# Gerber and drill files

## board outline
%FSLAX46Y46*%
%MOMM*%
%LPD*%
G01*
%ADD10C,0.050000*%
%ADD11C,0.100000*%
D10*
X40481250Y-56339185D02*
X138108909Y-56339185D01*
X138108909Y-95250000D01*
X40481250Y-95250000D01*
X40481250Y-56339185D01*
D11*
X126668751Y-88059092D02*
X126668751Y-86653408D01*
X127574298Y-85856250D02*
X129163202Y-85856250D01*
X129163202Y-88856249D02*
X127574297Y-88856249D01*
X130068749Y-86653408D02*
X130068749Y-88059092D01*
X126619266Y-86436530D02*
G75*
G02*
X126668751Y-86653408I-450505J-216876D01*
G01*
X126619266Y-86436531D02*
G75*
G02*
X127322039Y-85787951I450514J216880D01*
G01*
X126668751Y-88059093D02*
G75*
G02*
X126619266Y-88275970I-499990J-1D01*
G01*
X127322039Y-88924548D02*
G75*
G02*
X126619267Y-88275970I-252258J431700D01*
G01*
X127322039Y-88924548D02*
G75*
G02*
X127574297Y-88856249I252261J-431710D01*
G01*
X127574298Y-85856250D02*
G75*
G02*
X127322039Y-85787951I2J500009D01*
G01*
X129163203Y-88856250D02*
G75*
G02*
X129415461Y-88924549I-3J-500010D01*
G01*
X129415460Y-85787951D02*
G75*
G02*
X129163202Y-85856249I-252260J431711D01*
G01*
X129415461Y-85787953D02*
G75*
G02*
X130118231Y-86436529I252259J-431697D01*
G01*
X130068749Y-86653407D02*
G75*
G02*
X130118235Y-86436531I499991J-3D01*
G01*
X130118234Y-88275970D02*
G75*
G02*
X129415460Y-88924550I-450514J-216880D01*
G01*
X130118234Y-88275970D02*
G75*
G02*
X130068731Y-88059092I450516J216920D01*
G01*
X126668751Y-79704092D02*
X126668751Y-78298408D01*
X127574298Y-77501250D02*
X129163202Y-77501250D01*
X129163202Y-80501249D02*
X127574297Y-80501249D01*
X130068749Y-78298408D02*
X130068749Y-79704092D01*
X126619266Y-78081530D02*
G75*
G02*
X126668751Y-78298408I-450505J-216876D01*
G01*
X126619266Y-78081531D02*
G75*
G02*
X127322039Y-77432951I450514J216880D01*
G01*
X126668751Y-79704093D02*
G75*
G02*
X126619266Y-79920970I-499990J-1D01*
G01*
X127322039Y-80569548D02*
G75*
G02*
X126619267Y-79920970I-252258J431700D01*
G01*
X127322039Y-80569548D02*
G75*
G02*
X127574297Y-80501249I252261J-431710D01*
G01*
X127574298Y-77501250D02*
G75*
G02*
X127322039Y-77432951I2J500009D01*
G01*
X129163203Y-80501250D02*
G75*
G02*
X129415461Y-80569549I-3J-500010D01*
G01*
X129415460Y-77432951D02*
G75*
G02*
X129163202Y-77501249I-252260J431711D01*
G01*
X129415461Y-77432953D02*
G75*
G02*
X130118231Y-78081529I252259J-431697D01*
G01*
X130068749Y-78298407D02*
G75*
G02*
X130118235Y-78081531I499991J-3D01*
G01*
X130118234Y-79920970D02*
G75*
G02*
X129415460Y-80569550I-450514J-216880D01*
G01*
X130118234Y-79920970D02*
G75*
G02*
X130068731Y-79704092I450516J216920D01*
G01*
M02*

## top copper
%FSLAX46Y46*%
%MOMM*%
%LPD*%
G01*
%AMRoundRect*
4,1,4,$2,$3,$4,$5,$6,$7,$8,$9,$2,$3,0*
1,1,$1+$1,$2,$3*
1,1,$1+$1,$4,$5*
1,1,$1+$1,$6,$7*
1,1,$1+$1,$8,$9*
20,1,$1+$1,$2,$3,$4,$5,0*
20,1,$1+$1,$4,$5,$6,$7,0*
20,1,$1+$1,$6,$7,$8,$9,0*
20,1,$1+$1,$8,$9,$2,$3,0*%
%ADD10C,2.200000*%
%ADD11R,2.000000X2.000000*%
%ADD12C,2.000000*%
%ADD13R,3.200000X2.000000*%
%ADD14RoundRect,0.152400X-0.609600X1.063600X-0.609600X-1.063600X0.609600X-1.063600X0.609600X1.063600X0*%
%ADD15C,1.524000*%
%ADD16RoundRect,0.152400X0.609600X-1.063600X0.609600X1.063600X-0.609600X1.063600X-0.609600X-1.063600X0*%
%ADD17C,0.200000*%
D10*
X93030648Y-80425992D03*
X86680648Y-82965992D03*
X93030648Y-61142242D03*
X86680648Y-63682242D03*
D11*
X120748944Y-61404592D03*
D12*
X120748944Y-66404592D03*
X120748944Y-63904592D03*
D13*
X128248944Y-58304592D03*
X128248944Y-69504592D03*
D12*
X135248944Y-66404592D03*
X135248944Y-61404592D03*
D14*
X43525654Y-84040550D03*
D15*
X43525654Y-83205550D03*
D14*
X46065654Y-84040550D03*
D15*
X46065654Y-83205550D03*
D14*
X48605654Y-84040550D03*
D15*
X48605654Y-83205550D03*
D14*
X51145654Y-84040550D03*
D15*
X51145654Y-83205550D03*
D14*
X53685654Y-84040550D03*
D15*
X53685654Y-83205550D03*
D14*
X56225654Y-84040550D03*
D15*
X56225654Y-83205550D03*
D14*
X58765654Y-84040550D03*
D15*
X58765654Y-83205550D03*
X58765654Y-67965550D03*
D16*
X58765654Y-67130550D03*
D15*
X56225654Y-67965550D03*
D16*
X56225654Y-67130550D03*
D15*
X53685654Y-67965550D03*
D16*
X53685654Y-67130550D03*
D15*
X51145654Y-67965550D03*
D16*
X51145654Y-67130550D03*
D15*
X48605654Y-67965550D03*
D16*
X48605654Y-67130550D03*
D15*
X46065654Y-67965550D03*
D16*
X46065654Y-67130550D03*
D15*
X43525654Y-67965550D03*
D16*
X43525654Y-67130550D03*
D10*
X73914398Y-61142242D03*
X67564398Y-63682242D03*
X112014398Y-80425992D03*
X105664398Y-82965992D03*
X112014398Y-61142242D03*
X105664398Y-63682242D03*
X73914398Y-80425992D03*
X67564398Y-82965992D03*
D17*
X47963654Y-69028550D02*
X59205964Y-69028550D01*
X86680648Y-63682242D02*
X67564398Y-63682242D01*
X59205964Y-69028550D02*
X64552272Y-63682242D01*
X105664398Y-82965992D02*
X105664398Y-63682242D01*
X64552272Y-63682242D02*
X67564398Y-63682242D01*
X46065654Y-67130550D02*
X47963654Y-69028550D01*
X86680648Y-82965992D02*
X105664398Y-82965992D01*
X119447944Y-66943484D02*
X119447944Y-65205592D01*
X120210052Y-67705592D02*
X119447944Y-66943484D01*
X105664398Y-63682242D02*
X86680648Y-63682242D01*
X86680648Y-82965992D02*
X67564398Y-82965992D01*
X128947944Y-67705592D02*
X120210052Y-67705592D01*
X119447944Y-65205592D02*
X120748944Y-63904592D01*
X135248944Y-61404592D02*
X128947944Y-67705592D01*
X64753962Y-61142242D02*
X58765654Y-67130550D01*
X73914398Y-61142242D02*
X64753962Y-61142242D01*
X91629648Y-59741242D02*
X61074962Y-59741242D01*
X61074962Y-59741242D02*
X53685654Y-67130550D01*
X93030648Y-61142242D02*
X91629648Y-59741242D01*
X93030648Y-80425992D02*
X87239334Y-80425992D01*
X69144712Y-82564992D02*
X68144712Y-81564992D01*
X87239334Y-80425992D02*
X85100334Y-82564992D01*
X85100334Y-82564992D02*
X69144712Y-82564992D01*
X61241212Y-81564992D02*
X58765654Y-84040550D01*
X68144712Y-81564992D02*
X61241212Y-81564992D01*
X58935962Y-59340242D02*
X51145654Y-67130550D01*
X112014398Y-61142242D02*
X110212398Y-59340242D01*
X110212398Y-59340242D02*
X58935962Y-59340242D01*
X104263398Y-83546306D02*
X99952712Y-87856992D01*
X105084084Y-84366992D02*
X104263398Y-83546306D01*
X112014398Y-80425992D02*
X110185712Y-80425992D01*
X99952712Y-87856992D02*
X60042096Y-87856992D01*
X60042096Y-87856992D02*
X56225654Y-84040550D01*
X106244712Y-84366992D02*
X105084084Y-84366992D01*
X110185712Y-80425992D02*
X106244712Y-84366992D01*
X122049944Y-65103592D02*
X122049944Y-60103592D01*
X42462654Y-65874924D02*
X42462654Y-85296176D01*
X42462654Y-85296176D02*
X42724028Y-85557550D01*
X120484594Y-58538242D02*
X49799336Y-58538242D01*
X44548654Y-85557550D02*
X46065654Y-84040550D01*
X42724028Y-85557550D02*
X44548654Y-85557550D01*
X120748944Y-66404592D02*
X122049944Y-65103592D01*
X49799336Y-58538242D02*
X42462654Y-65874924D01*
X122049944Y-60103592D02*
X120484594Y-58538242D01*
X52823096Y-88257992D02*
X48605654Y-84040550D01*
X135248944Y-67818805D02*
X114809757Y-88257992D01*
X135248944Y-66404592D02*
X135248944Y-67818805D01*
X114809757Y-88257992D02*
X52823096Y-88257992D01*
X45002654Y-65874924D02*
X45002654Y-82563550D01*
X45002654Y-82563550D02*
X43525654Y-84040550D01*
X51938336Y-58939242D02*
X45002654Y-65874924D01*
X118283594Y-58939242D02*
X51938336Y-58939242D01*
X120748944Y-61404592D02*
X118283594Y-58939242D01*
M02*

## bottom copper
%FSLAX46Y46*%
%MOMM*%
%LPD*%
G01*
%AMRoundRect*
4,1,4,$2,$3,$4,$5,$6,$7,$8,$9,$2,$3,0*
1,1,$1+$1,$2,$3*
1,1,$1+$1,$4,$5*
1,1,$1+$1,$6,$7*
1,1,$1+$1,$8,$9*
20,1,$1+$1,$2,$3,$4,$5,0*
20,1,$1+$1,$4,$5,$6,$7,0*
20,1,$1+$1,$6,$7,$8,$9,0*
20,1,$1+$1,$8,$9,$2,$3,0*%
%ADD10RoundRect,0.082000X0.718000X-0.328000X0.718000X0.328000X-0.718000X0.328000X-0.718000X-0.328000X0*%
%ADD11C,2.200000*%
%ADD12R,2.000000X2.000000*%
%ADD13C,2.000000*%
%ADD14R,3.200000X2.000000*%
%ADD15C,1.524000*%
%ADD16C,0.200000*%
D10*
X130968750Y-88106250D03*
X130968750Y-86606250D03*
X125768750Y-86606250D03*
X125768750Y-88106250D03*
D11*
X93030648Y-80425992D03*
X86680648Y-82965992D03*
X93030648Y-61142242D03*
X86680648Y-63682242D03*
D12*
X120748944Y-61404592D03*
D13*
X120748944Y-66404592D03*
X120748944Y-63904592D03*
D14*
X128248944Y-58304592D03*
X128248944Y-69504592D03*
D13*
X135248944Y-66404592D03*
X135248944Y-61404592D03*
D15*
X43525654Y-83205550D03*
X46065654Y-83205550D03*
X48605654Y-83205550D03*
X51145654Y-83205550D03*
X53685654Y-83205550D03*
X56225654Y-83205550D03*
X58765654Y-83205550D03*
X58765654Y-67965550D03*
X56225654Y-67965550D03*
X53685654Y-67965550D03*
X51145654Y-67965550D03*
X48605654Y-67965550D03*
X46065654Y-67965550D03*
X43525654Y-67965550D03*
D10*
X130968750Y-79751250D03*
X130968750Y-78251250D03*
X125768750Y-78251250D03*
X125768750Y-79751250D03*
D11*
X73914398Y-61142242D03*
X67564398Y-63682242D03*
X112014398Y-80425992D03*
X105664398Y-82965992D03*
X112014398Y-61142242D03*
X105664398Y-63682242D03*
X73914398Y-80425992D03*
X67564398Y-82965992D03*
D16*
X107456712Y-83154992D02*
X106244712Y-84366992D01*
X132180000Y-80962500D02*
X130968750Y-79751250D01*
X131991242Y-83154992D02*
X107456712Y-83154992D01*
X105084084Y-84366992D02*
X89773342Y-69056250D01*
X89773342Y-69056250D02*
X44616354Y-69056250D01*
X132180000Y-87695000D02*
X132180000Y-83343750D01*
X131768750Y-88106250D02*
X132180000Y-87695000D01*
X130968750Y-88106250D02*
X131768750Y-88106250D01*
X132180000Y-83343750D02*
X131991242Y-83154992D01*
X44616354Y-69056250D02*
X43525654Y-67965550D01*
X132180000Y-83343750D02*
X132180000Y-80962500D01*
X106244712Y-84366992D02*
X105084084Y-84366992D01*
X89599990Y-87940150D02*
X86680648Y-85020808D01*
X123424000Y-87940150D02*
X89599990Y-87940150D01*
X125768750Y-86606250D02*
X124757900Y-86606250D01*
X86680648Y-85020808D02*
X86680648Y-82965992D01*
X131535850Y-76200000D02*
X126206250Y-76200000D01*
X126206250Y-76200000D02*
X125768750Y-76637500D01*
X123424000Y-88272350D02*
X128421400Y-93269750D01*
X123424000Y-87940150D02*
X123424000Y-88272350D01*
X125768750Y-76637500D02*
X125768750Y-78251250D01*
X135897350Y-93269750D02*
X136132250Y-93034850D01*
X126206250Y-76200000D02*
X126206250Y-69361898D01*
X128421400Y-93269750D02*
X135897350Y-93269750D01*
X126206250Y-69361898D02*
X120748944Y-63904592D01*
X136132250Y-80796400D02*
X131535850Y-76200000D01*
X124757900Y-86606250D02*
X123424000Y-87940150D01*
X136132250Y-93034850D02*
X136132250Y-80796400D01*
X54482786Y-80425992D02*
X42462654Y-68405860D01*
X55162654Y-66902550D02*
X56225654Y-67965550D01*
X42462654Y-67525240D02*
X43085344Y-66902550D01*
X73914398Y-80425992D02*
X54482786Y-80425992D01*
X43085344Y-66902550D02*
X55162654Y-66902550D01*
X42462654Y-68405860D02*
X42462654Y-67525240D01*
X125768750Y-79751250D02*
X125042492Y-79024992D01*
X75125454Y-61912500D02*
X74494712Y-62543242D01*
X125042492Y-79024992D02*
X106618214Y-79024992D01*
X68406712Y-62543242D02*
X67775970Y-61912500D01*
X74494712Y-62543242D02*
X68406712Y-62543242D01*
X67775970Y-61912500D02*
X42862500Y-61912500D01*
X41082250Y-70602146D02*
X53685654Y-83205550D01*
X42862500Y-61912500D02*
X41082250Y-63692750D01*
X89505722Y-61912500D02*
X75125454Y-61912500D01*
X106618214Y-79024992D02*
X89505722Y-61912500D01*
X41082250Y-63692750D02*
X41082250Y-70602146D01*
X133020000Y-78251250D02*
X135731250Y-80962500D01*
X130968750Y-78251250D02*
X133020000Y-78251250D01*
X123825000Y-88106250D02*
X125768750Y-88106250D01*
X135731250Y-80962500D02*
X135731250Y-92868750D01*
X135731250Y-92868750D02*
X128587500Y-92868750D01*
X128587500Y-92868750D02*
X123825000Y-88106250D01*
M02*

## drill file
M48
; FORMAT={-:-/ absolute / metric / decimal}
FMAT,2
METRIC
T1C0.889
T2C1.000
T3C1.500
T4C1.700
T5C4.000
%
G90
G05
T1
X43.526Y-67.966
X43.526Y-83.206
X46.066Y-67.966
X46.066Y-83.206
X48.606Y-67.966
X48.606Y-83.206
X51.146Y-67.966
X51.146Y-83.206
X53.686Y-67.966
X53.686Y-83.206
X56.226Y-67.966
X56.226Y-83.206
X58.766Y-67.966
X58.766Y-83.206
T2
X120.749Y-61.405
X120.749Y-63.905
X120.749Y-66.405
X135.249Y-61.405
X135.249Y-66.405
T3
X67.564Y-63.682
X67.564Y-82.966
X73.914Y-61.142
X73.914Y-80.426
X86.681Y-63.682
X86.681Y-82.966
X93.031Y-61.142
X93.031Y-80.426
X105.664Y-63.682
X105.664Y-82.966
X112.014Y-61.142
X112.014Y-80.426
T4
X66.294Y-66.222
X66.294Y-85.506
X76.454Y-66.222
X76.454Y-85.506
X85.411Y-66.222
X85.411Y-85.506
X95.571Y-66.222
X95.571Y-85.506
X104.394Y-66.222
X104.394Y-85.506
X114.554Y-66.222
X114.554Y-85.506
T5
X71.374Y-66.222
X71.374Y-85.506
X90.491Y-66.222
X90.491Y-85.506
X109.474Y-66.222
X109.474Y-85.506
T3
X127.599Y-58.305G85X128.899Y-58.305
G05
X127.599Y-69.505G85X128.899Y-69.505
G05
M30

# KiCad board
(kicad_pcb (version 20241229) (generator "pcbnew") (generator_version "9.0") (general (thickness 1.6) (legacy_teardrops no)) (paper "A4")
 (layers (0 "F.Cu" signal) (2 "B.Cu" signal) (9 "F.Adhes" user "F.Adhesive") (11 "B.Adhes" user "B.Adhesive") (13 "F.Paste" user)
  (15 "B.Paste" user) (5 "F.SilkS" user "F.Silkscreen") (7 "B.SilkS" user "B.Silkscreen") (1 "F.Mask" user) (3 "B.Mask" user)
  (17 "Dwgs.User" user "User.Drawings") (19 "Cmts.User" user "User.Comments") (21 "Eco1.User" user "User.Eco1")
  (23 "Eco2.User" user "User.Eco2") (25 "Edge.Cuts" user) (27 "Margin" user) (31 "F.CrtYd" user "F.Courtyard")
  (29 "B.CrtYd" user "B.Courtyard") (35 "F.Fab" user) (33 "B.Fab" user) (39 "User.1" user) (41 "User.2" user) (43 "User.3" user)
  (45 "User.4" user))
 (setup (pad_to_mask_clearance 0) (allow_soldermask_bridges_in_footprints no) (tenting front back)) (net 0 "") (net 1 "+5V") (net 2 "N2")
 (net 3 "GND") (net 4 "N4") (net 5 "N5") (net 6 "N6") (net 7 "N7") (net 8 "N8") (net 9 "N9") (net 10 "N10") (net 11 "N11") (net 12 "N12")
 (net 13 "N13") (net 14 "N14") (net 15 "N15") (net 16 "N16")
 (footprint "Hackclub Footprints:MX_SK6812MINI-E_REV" (layer "F.Cu") (at 128.36875 82.27625)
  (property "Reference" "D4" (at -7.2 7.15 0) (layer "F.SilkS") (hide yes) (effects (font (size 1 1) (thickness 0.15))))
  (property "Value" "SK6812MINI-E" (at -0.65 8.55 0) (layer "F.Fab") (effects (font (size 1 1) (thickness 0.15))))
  (fp_line (start -1.699999 5.782842) (end -1.699999 4.377158) (stroke (width 0.1) (type solid)) (layer "Edge.Cuts"))
  (fp_line (start -0.794452 3.58) (end 0.794452 3.58) (stroke (width 0.1) (type solid)) (layer "Edge.Cuts"))
  (fp_line (start 0.794452 6.579999) (end -0.794453 6.579999) (stroke (width 0.1) (type solid)) (layer "Edge.Cuts"))
  (fp_line (start 1.699999 4.377158) (end 1.699999 5.782842) (stroke (width 0.1) (type solid)) (layer "Edge.Cuts"))
  (fp_arc (start -1.749484 4.16028) (mid -1.712527 4.265932) (end -1.699999 4.377158) (stroke (width 0.1) (type solid)) (layer "Edge.Cuts"))
  (fp_arc (start -1.749484 4.160281) (mid -1.638072 3.575965) (end -1.046711 3.511701) (stroke (width 0.1) (type solid)) (layer "Edge.Cuts"))
  (fp_arc (start -1.699999 5.782843) (mid -1.712527 5.894068) (end -1.749484 5.99972) (stroke (width 0.1) (type solid)) (layer "Edge.Cuts"))
  (fp_arc (start -1.046711 6.648298) (mid -1.638071 6.584034) (end -1.749484 5.99972) (stroke (width 0.1) (type solid)) (layer "Edge.Cuts"))
  (fp_arc (start -1.046711 6.648298) (mid -0.925123 6.597376) (end -0.794453 6.579999) (stroke (width 0.1) (type solid)) (layer "Edge.Cuts"))
  (fp_arc (start -0.794452 3.58) (mid -0.925123 3.562623) (end -1.046711 3.511701) (stroke (width 0.1) (type solid)) (layer "Edge.Cuts"))
  (fp_arc (start 0.794453 6.58) (mid 0.925123 6.597377) (end 1.046711 6.648299) (stroke (width 0.1) (type solid)) (layer "Edge.Cuts"))
  (fp_arc (start 1.04671 3.511701) (mid 0.925122 3.562623) (end 0.794452 3.58) (stroke (width 0.1) (type solid)) (layer "Edge.Cuts"))
  (fp_arc (start 1.046711 3.511703) (mid 1.63807 3.575966) (end 1.749484 4.16028) (stroke (width 0.1) (type solid)) (layer "Edge.Cuts"))
  (fp_arc (start 1.699999 4.377157) (mid 1.712527 4.265932) (end 1.749484 4.16028) (stroke (width 0.1) (type solid)) (layer "Edge.Cuts"))
  (fp_arc (start 1.749484 5.99972) (mid 1.638071 6.584035) (end 1.046711 6.648299) (stroke (width 0.1) (type solid)) (layer "Edge.Cuts"))
  (fp_arc (start 1.749484 5.99972) (mid 1.712527 5.894068) (end 1.699999 5.782842) (stroke (width 0.1) (type solid)) (layer "Edge.Cuts"))
  (pad "1" smd roundrect (at 2.6 5.83 90) (size 0.82 1.6) (layers "B.Cu" "B.Mask" "B.Paste") (roundrect_rratio 0.1) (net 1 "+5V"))
  (pad "2" smd roundrect (at 2.6 4.33 90) (size 0.82 1.6) (layers "B.Cu" "B.Mask" "B.Paste") (roundrect_rratio 0.1) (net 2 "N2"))
  (pad "3" smd roundrect (at -2.6 4.33 90) (size 0.82 1.6) (layers "B.Cu" "B.Mask" "B.Paste") (roundrect_rratio 0.1) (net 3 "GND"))
  (pad "4" smd roundrect (at -2.6 5.83 90) (size 0.82 1.6) (layers "B.Cu" "B.Mask" "B.Paste") (roundrect_rratio 0.1) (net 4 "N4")))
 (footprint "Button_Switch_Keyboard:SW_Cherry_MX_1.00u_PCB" (layer "F.Cu") (at 93.030648 80.425992)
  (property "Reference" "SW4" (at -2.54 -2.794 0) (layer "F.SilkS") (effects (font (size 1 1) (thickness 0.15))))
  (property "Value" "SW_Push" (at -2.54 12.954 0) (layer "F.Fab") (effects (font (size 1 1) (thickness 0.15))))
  (pad "" np_thru_hole circle (at -7.62 5.08) (size 1.7 1.7) (drill 1.7) (layers "*.Cu" "*.Mask"))
  (pad "" np_thru_hole circle (at -2.54 5.08) (size 4 4) (drill 4) (layers "*.Cu" "*.Mask"))
  (pad "" np_thru_hole circle (at 2.54 5.08) (size 1.7 1.7) (drill 1.7) (layers "*.Cu" "*.Mask"))
  (pad "1" thru_hole circle (at 0 0) (size 2.2 2.2) (drill 1.5) (layers "*.Cu" "*.Mask") (remove_unused_layers no) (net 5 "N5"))
  (pad "2" thru_hole circle (at -6.35 2.54) (size 2.2 2.2) (drill 1.5) (layers "*.Cu" "*.Mask") (remove_unused_layers no) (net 3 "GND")))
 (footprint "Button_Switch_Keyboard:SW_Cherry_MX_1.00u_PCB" (layer "F.Cu") (at 93.030648 61.142242)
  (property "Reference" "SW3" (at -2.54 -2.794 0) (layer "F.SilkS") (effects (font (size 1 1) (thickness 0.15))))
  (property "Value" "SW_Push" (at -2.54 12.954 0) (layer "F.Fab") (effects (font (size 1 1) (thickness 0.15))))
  (pad "" np_thru_hole circle (at -7.62 5.08) (size 1.7 1.7) (drill 1.7) (layers "*.Cu" "*.Mask"))
  (pad "" np_thru_hole circle (at -2.54 5.08) (size 4 4) (drill 4) (layers "*.Cu" "*.Mask"))
  (pad "" np_thru_hole circle (at 2.54 5.08) (size 1.7 1.7) (drill 1.7) (layers "*.Cu" "*.Mask"))
  (pad "1" thru_hole circle (at 0 0) (size 2.2 2.2) (drill 1.5) (layers "*.Cu" "*.Mask") (remove_unused_layers no) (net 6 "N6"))
  (pad "2" thru_hole circle (at -6.35 2.54) (size 2.2 2.2) (drill 1.5) (layers "*.Cu" "*.Mask") (remove_unused_layers no) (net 3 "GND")))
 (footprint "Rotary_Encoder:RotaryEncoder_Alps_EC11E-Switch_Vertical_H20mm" (layer "F.Cu") (at 120.748944 61.404592)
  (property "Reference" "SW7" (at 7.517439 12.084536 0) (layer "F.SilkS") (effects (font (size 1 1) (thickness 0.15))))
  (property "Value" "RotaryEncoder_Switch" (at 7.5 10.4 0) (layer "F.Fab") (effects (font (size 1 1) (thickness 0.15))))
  (pad "A" thru_hole rect (at 0 0) (size 2 2) (drill 1) (layers "*.Cu" "*.Mask") (remove_unused_layers no) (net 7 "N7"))
  (pad "B" thru_hole circle (at 0 5) (size 2 2) (drill 1) (layers "*.Cu" "*.Mask") (remove_unused_layers no) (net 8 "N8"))
  (pad "C" thru_hole circle (at 0 2.5) (size 2 2) (drill 1) (layers "*.Cu" "*.Mask") (remove_unused_layers no) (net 3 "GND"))
  (pad "MP" thru_hole rect (at 7.5 -3.1) (size 3.2 2) (drill oval 2.8 1.5) (layers "*.Cu" "*.Mask") (remove_unused_layers no))
  (pad "MP" thru_hole rect (at 7.5 8.1) (size 3.2 2) (drill oval 2.8 1.5) (layers "*.Cu" "*.Mask") (remove_unused_layers no))
  (pad "S1" thru_hole circle (at 14.5 5) (size 2 2) (drill 1) (layers "*.Cu" "*.Mask") (remove_unused_layers no) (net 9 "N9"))
  (pad "S2" thru_hole circle (at 14.5 0) (size 2 2) (drill 1) (layers "*.Cu" "*.Mask") (remove_unused_layers no) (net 3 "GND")))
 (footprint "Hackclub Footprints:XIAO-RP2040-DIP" (layer "F.Cu") (at 51.145654 75.58555 90)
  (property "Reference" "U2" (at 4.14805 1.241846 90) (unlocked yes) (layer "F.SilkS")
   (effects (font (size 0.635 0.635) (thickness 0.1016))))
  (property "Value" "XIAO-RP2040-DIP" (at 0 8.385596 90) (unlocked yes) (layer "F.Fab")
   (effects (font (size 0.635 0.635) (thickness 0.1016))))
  (pad "1" smd roundrect (at -8.455 -7.62 270) (size 2.432 1.524) (layers "F.Cu" "F.Mask") (roundrect_rratio 0.1) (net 7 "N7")
   (thermal_bridge_angle 45))
  (pad "1" thru_hole circle (at -7.62 -7.62 270) (size 1.524 1.524) (drill 0.889) (layers "*.Cu" "*.Mask") (remove_unused_layers no)
   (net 7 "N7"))
  (pad "2" smd roundrect (at -8.455 -5.08 270) (size 2.432 1.524) (layers "F.Cu" "F.Mask") (roundrect_rratio 0.1) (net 8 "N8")
   (thermal_bridge_angle 45))
  (pad "2" thru_hole circle (at -7.62 -5.08 270) (size 1.524 1.524) (drill 0.889) (layers "*.Cu" "*.Mask") (remove_unused_layers no)
   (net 8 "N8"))
  (pad "3" smd roundrect (at -8.455 -2.54 270) (size 2.432 1.524) (layers "F.Cu" "F.Mask") (roundrect_rratio 0.1) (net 9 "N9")
   (thermal_bridge_angle 45))
  (pad "3" thru_hole circle (at -7.62 -2.54 270) (size 1.524 1.524) (drill 0.889) (layers "*.Cu" "*.Mask") (remove_unused_layers no)
   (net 9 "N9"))
  (pad "4" smd roundrect (at -8.455 0 270) (size 2.432 1.524) (layers "F.Cu" "F.Mask") (roundrect_rratio 0.1) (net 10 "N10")
   (thermal_bridge_angle 45))
  (pad "4" thru_hole circle (at -7.62 0 270) (size 1.524 1.524) (drill 0.889) (layers "*.Cu" "*.Mask") (remove_unused_layers no)
   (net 10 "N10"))
  (pad "5" smd roundrect (at -8.455 2.54 270) (size 2.432 1.524) (layers "F.Cu" "F.Mask") (roundrect_rratio 0.1) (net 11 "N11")
   (thermal_bridge_angle 45))
  (pad "5" thru_hole circle (at -7.62 2.54 270) (size 1.524 1.524) (drill 0.889) (layers "*.Cu" "*.Mask") (remove_unused_layers no)
   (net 11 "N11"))
  (pad "6" smd roundrect (at -8.455 5.08 270) (size 2.432 1.524) (layers "F.Cu" "F.Mask") (roundrect_rratio 0.1) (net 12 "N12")
   (thermal_bridge_angle 45))
  (pad "6" thru_hole circle (at -7.62 5.08 270) (size 1.524 1.524) (drill 0.889) (layers "*.Cu" "*.Mask") (remove_unused_layers no)
   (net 12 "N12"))
  (pad "7" smd roundrect (at -8.455 7.62 270) (size 2.432 1.524) (layers "F.Cu" "F.Mask") (roundrect_rratio 0.1) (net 5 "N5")
   (thermal_bridge_angle 45))
  (pad "7" thru_hole circle (at -7.62 7.62 270) (size 1.524 1.524) (drill 0.889) (layers "*.Cu" "*.Mask") (remove_unused_layers no)
   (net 5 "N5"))
  (pad "8" thru_hole circle (at 7.62 7.62 90) (size 1.524 1.524) (drill 0.889) (layers "*.Cu" "*.Mask") (remove_unused_layers no)
   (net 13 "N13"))
  (pad "8" smd roundrect (at 8.455 7.62 90) (size 2.432 1.524) (layers "F.Cu" "F.Mask") (roundrect_rratio 0.1) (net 13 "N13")
   (thermal_bridge_angle 45))
  (pad "9" thru_hole circle (at 7.62 5.08 90) (size 1.524 1.524) (drill 0.889) (layers "*.Cu" "*.Mask") (remove_unused_layers no)
   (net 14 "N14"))
  (pad "9" smd roundrect (at 8.455 5.08 90) (size 2.432 1.524) (layers "F.Cu" "F.Mask") (roundrect_rratio 0.1) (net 14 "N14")
   (thermal_bridge_angle 45))
  (pad "10" thru_hole circle (at 7.62 2.54 90) (size 1.524 1.524) (drill 0.889) (layers "*.Cu" "*.Mask") (remove_unused_layers no)
   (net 6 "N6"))
  (pad "10" smd roundrect (at 8.455 2.54 90) (size 2.432 1.524) (layers "F.Cu" "F.Mask") (roundrect_rratio 0.1) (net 6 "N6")
   (thermal_bridge_angle 45))
  (pad "11" thru_hole circle (at 7.62 0 90) (size 1.524 1.524) (drill 0.889) (layers "*.Cu" "*.Mask") (remove_unused_layers no)
   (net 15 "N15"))
  (pad "11" smd roundrect (at 8.455 0 90) (size 2.432 1.524) (layers "F.Cu" "F.Mask") (roundrect_rratio 0.1) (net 15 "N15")
   (thermal_bridge_angle 45))
  (pad "12" thru_hole circle (at 7.62 -2.54 90) (size 1.524 1.524) (drill 0.889) (layers "*.Cu" "*.Mask") (remove_unused_layers no)
   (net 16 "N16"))
  (pad "12" smd roundrect (at 8.455 -2.54 90) (size 2.432 1.524) (layers "F.Cu" "F.Mask") (roundrect_rratio 0.1) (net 16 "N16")
   (thermal_bridge_angle 45))
  (pad "13" thru_hole circle (at 7.62 -5.08 90) (size 1.524 1.524) (drill 0.889) (layers "*.Cu" "*.Mask") (remove_unused_layers no)
   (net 3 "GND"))
  (pad "13" smd roundrect (at 8.455 -5.08 90) (size 2.432 1.524) (layers "F.Cu" "F.Mask") (roundrect_rratio 0.1) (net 3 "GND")
   (thermal_bridge_angle 45))
  (pad "14" thru_hole circle (at 7.62 -7.62 90) (size 1.524 1.524) (drill 0.889) (layers "*.Cu" "*.Mask") (remove_unused_layers no)
   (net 1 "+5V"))
  (pad "14" smd roundrect (at 8.455 -7.62 90) (size 2.432 1.524) (layers "F.Cu" "F.Mask") (roundrect_rratio 0.1) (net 1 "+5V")
   (thermal_bridge_angle 45)))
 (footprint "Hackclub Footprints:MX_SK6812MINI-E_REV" (layer "F.Cu") (at 128.36875 73.92125)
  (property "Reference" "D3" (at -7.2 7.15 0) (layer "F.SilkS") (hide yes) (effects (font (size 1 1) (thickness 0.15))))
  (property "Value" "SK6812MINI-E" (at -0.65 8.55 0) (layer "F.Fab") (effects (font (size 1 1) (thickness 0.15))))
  (fp_line (start -1.699999 5.782842) (end -1.699999 4.377158) (stroke (width 0.1) (type solid)) (layer "Edge.Cuts"))
  (fp_line (start -0.794452 3.58) (end 0.794452 3.58) (stroke (width 0.1) (type solid)) (layer "Edge.Cuts"))
  (fp_line (start 0.794452 6.579999) (end -0.794453 6.579999) (stroke (width 0.1) (type solid)) (layer "Edge.Cuts"))
  (fp_line (start 1.699999 4.377158) (end 1.699999 5.782842) (stroke (width 0.1) (type solid)) (layer "Edge.Cuts"))
  (fp_arc (start -1.749484 4.16028) (mid -1.712527 4.265932) (end -1.699999 4.377158) (stroke (width 0.1) (type solid)) (layer "Edge.Cuts"))
  (fp_arc (start -1.749484 4.160281) (mid -1.638072 3.575965) (end -1.046711 3.511701) (stroke (width 0.1) (type solid)) (layer "Edge.Cuts"))
  (fp_arc (start -1.699999 5.782843) (mid -1.712527 5.894068) (end -1.749484 5.99972) (stroke (width 0.1) (type solid)) (layer "Edge.Cuts"))
  (fp_arc (start -1.046711 6.648298) (mid -1.638071 6.584034) (end -1.749484 5.99972) (stroke (width 0.1) (type solid)) (layer "Edge.Cuts"))
  (fp_arc (start -1.046711 6.648298) (mid -0.925123 6.597376) (end -0.794453 6.579999) (stroke (width 0.1) (type solid)) (layer "Edge.Cuts"))
  (fp_arc (start -0.794452 3.58) (mid -0.925123 3.562623) (end -1.046711 3.511701) (stroke (width 0.1) (type solid)) (layer "Edge.Cuts"))
  (fp_arc (start 0.794453 6.58) (mid 0.925123 6.597377) (end 1.046711 6.648299) (stroke (width 0.1) (type solid)) (layer "Edge.Cuts"))
  (fp_arc (start 1.04671 3.511701) (mid 0.925122 3.562623) (end 0.794452 3.58) (stroke (width 0.1) (type solid)) (layer "Edge.Cuts"))
  (fp_arc (start 1.046711 3.511703) (mid 1.63807 3.575966) (end 1.749484 4.16028) (stroke (width 0.1) (type solid)) (layer "Edge.Cuts"))
  (fp_arc (start 1.699999 4.377157) (mid 1.712527 4.265932) (end 1.749484 4.16028) (stroke (width 0.1) (type solid)) (layer "Edge.Cuts"))
  (fp_arc (start 1.749484 5.99972) (mid 1.638071 6.584035) (end 1.046711 6.648299) (stroke (width 0.1) (type solid)) (layer "Edge.Cuts"))
  (fp_arc (start 1.749484 5.99972) (mid 1.712527 5.894068) (end 1.699999 5.782842) (stroke (width 0.1) (type solid)) (layer "Edge.Cuts"))
  (pad "1" smd roundrect (at 2.6 5.83 90) (size 0.82 1.6) (layers "B.Cu" "B.Mask" "B.Paste") (roundrect_rratio 0.1) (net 1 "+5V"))
  (pad "2" smd roundrect (at 2.6 4.33 90) (size 0.82 1.6) (layers "B.Cu" "B.Mask" "B.Paste") (roundrect_rratio 0.1) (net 4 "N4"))
  (pad "3" smd roundrect (at -2.6 4.33 90) (size 0.82 1.6) (layers "B.Cu" "B.Mask" "B.Paste") (roundrect_rratio 0.1) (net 3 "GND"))
  (pad "4" smd roundrect (at -2.6 5.83 90) (size 0.82 1.6) (layers "B.Cu" "B.Mask" "B.Paste") (roundrect_rratio 0.1) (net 11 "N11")))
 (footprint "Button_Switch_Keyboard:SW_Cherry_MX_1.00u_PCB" (layer "F.Cu") (at 73.914398 61.142242)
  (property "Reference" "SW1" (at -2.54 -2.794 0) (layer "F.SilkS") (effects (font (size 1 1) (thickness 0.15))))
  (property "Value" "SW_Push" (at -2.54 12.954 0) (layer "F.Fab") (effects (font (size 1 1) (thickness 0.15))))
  (pad "" np_thru_hole circle (at -7.62 5.08) (size 1.7 1.7) (drill 1.7) (layers "*.Cu" "*.Mask"))
  (pad "" np_thru_hole circle (at -2.54 5.08) (size 4 4) (drill 4) (layers "*.Cu" "*.Mask"))
  (pad "" np_thru_hole circle (at 2.54 5.08) (size 1.7 1.7) (drill 1.7) (layers "*.Cu" "*.Mask"))
  (pad "1" thru_hole circle (at 0 0) (size 2.2 2.2) (drill 1.5) (layers "*.Cu" "*.Mask") (remove_unused_layers no) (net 13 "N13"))
  (pad "2" thru_hole circle (at -6.35 2.54) (size 2.2 2.2) (drill 1.5) (layers "*.Cu" "*.Mask") (remove_unused_layers no) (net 3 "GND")))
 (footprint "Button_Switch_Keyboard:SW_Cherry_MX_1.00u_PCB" (layer "F.Cu") (at 112.014398 80.425992)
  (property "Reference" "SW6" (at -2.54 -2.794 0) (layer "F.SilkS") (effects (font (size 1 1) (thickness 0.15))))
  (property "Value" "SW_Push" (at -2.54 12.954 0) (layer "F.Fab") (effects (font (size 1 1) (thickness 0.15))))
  (pad "" np_thru_hole circle (at -7.62 5.08) (size 1.7 1.7) (drill 1.7) (layers "*.Cu" "*.Mask"))
  (pad "" np_thru_hole circle (at -2.54 5.08) (size 4 4) (drill 4) (layers "*.Cu" "*.Mask"))
  (pad "" np_thru_hole circle (at 2.54 5.08) (size 1.7 1.7) (drill 1.7) (layers "*.Cu" "*.Mask"))
  (pad "1" thru_hole circle (at 0 0) (size 2.2 2.2) (drill 1.5) (layers "*.Cu" "*.Mask") (remove_unused_layers no) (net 12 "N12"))
  (pad "2" thru_hole circle (at -6.35 2.54) (size 2.2 2.2) (drill 1.5) (layers "*.Cu" "*.Mask") (remove_unused_layers no) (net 3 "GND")))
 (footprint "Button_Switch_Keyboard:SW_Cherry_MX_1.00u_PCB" (layer "F.Cu") (at 112.014398 61.142242)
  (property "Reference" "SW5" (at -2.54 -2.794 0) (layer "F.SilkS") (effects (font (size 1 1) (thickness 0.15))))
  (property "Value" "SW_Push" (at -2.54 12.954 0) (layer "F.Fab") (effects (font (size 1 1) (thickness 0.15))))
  (pad "" np_thru_hole circle (at -7.62 5.08) (size 1.7 1.7) (drill 1.7) (layers "*.Cu" "*.Mask"))
  (pad "" np_thru_hole circle (at -2.54 5.08) (size 4 4) (drill 4) (layers "*.Cu" "*.Mask"))
  (pad "" np_thru_hole circle (at 2.54 5.08) (size 1.7 1.7) (drill 1.7) (layers "*.Cu" "*.Mask"))
  (pad "1" thru_hole circle (at 0 0) (size 2.2 2.2) (drill 1.5) (layers "*.Cu" "*.Mask") (remove_unused_layers no) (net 15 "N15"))
  (pad "2" thru_hole circle (at -6.35 2.54) (size 2.2 2.2) (drill 1.5) (layers "*.Cu" "*.Mask") (remove_unused_layers no) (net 3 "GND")))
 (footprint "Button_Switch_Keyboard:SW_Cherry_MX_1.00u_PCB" (layer "F.Cu") (at 73.914398 80.425992)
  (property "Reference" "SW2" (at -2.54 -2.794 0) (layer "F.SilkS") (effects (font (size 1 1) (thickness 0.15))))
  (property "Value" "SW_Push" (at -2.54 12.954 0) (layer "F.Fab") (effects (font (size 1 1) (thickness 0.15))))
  (pad "" np_thru_hole circle (at -7.62 5.08) (size 1.7 1.7) (drill 1.7) (layers "*.Cu" "*.Mask"))
  (pad "" np_thru_hole circle (at -2.54 5.08) (size 4 4) (drill 4) (layers "*.Cu" "*.Mask"))
  (pad "" np_thru_hole circle (at 2.54 5.08) (size 1.7 1.7) (drill 1.7) (layers "*.Cu" "*.Mask"))
  (pad "1" thru_hole circle (at 0 0) (size 2.2 2.2) (drill 1.5) (layers "*.Cu" "*.Mask") (remove_unused_layers no) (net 14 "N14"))
  (pad "2" thru_hole circle (at -6.35 2.54) (size 2.2 2.2) (drill 1.5) (layers "*.Cu" "*.Mask") (remove_unused_layers no) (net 3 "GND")))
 (gr_rect (start 40.48125 56.339185) (end 138.108909 95.25) (stroke (width 0.05) (type default)) (fill no) (layer "Edge.Cuts"))
 (segment (start 107.456712 83.154992) (end 106.244712 84.366992) (width 0.2) (layer "B.Cu") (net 1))
 (segment (start 132.18 80.9625) (end 130.96875 79.75125) (width 0.2) (layer "B.Cu") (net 1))
 (segment (start 131.991242 83.154992) (end 107.456712 83.154992) (width 0.2) (layer "B.Cu") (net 1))
 (segment (start 105.084084 84.366992) (end 89.773342 69.05625) (width 0.2) (layer "B.Cu") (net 1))
 (segment (start 89.773342 69.05625) (end 44.616354 69.05625) (width 0.2) (layer "B.Cu") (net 1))
 (segment (start 132.18 87.695) (end 132.18 83.34375) (width 0.2) (layer "B.Cu") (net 1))
 (segment (start 131.76875 88.10625) (end 132.18 87.695) (width 0.2) (layer "B.Cu") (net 1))
 (segment (start 130.96875 88.10625) (end 131.76875 88.10625) (width 0.2) (layer "B.Cu") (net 1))
 (segment (start 132.18 83.34375) (end 131.991242 83.154992) (width 0.2) (layer "B.Cu") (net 1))
 (segment (start 44.616354 69.05625) (end 43.525654 67.96555) (width 0.2) (layer "B.Cu") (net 1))
 (segment (start 132.18 83.34375) (end 132.18 80.9625) (width 0.2) (layer "B.Cu") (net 1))
 (segment (start 106.244712 84.366992) (end 105.084084 84.366992) (width 0.2) (layer "B.Cu") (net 1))
 (segment (start 47.963654 69.02855) (end 59.205964 69.02855) (width 0.2) (layer "F.Cu") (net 3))
 (segment (start 86.680648 63.682242) (end 67.564398 63.682242) (width 0.2) (layer "F.Cu") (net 3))
 (segment (start 59.205964 69.02855) (end 64.552272 63.682242) (width 0.2) (layer "F.Cu") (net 3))
 (segment (start 105.664398 82.965992) (end 105.664398 63.682242) (width 0.2) (layer "F.Cu") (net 3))
 (segment (start 64.552272 63.682242) (end 67.564398 63.682242) (width 0.2) (layer "F.Cu") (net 3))
 (segment (start 46.065654 67.13055) (end 47.963654 69.02855) (width 0.2) (layer "F.Cu") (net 3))
 (segment (start 86.680648 82.965992) (end 105.664398 82.965992) (width 0.2) (layer "F.Cu") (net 3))
 (segment (start 119.447944 66.943484) (end 119.447944 65.205592) (width 0.2) (layer "F.Cu") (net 3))
 (segment (start 120.210052 67.705592) (end 119.447944 66.943484) (width 0.2) (layer "F.Cu") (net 3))
 (segment (start 105.664398 63.682242) (end 86.680648 63.682242) (width 0.2) (layer "F.Cu") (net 3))
 (segment (start 86.680648 82.965992) (end 67.564398 82.965992) (width 0.2) (layer "F.Cu") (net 3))
 (segment (start 128.947944 67.705592) (end 120.210052 67.705592) (width 0.2) (layer "F.Cu") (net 3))
 (segment (start 119.447944 65.205592) (end 120.748944 63.904592) (width 0.2) (layer "F.Cu") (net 3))
 (segment (start 135.248944 61.404592) (end 128.947944 67.705592) (width 0.2) (layer "F.Cu") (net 3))
 (segment (start 89.59999 87.94015) (end 86.680648 85.020808) (width 0.2) (layer "B.Cu") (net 3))
 (segment (start 123.424 87.94015) (end 89.59999 87.94015) (width 0.2) (layer "B.Cu") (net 3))
 (segment (start 125.76875 86.60625) (end 124.7579 86.60625) (width 0.2) (layer "B.Cu") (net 3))
 (segment (start 86.680648 85.020808) (end 86.680648 82.965992) (width 0.2) (layer "B.Cu") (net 3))
 (segment (start 131.53585 76.2) (end 126.20625 76.2) (width 0.2) (layer "B.Cu") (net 3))
 (segment (start 126.20625 76.2) (end 125.76875 76.6375) (width 0.2) (layer "B.Cu") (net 3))
 (segment (start 123.424 88.27235) (end 128.4214 93.26975) (width 0.2) (layer "B.Cu") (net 3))
 (segment (start 123.424 87.94015) (end 123.424 88.27235) (width 0.2) (layer "B.Cu") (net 3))
 (segment (start 125.76875 76.6375) (end 125.76875 78.25125) (width 0.2) (layer "B.Cu") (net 3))
 (segment (start 135.89735 93.26975) (end 136.13225 93.03485) (width 0.2) (layer "B.Cu") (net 3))
 (segment (start 126.20625 76.2) (end 126.20625 69.361898) (width 0.2) (layer "B.Cu") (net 3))
 (segment (start 128.4214 93.26975) (end 135.89735 93.26975) (width 0.2) (layer "B.Cu") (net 3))
 (segment (start 126.20625 69.361898) (end 120.748944 63.904592) (width 0.2) (layer "B.Cu") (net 3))
 (segment (start 136.13225 80.7964) (end 131.53585 76.2) (width 0.2) (layer "B.Cu") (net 3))
 (segment (start 124.7579 86.60625) (end 123.424 87.94015) (width 0.2) (layer "B.Cu") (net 3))
 (segment (start 136.13225 93.03485) (end 136.13225 80.7964) (width 0.2) (layer "B.Cu") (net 3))
 (segment (start 64.753962 61.142242) (end 58.765654 67.13055) (width 0.2) (layer "F.Cu") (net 13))
 (segment (start 73.914398 61.142242) (end 64.753962 61.142242) (width 0.2) (layer "F.Cu") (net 13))
 (segment (start 54.482786 80.425992) (end 42.462654 68.40586) (width 0.2) (layer "B.Cu") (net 14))
 (segment (start 55.162654 66.90255) (end 56.225654 67.96555) (width 0.2) (layer "B.Cu") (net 14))
 (segment (start 42.462654 67.52524) (end 43.085344 66.90255) (width 0.2) (layer "B.Cu") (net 14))
 (segment (start 73.914398 80.425992) (end 54.482786 80.425992) (width 0.2) (layer "B.Cu") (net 14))
 (segment (start 43.085344 66.90255) (end 55.162654 66.90255) (width 0.2) (layer "B.Cu") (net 14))
 (segment (start 42.462654 68.40586) (end 42.462654 67.52524) (width 0.2) (layer "B.Cu") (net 14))
 (segment (start 91.629648 59.741242) (end 61.074962 59.741242) (width 0.2) (layer "F.Cu") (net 6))
 (segment (start 61.074962 59.741242) (end 53.685654 67.13055) (width 0.2) (layer "F.Cu") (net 6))
 (segment (start 93.030648 61.142242) (end 91.629648 59.741242) (width 0.2) (layer "F.Cu") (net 6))
 (segment (start 93.030648 80.425992) (end 87.239334 80.425992) (width 0.2) (layer "F.Cu") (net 5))
 (segment (start 69.144712 82.564992) (end 68.144712 81.564992) (width 0.2) (layer "F.Cu") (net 5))
 (segment (start 87.239334 80.425992) (end 85.100334 82.564992) (width 0.2) (layer "F.Cu") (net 5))
 (segment (start 85.100334 82.564992) (end 69.144712 82.564992) (width 0.2) (layer "F.Cu") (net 5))
 (segment (start 61.241212 81.564992) (end 58.765654 84.04055) (width 0.2) (layer "F.Cu") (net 5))
 (segment (start 68.144712 81.564992) (end 61.241212 81.564992) (width 0.2) (layer "F.Cu") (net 5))
 (segment (start 58.935962 59.340242) (end 51.145654 67.13055) (width 0.2) (layer "F.Cu") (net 15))
 (segment (start 112.014398 61.142242) (end 110.212398 59.340242) (width 0.2) (layer "F.Cu") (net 15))
 (segment (start 110.212398 59.340242) (end 58.935962 59.340242) (width 0.2) (layer "F.Cu") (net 15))
 (segment (start 104.263398 83.546306) (end 99.952712 87.856992) (width 0.2) (layer "F.Cu") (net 12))
 (segment (start 105.084084 84.366992) (end 104.263398 83.546306) (width 0.2) (layer "F.Cu") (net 12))
 (segment (start 112.014398 80.425992) (end 110.185712 80.425992) (width 0.2) (layer "F.Cu") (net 12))
 (segment (start 99.952712 87.856992) (end 60.042096 87.856992) (width 0.2) (layer "F.Cu") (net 12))
 (segment (start 60.042096 87.856992) (end 56.225654 84.04055) (width 0.2) (layer "F.Cu") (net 12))
 (segment (start 106.244712 84.366992) (end 105.084084 84.366992) (width 0.2) (layer "F.Cu") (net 12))
 (segment (start 110.185712 80.425992) (end 106.244712 84.366992) (width 0.2) (layer "F.Cu") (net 12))
 (segment (start 122.049944 65.103592) (end 122.049944 60.103592) (width 0.2) (layer "F.Cu") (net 8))
 (segment (start 42.462654 65.874924) (end 42.462654 85.296176) (width 0.2) (layer "F.Cu") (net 8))
 (segment (start 42.462654 85.296176) (end 42.724028 85.55755) (width 0.2) (layer "F.Cu") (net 8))
 (segment (start 120.484594 58.538242) (end 49.799336 58.538242) (width 0.2) (layer "F.Cu") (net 8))
 (segment (start 44.548654 85.55755) (end 46.065654 84.04055) (width 0.2) (layer "F.Cu") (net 8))
 (segment (start 42.724028 85.55755) (end 44.548654 85.55755) (width 0.2) (layer "F.Cu") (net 8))
 (segment (start 120.748944 66.404592) (end 122.049944 65.103592) (width 0.2) (layer "F.Cu") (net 8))
 (segment (start 49.799336 58.538242) (end 42.462654 65.874924) (width 0.2) (layer "F.Cu") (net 8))
 (segment (start 122.049944 60.103592) (end 120.484594 58.538242) (width 0.2) (layer "F.Cu") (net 8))
 (segment (start 52.823096 88.257992) (end 48.605654 84.04055) (width 0.2) (layer "F.Cu") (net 9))
 (segment (start 135.248944 67.818805) (end 114.809757 88.257992) (width 0.2) (layer "F.Cu") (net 9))
 (segment (start 135.248944 66.404592) (end 135.248944 67.818805) (width 0.2) (layer "F.Cu") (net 9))
 (segment (start 114.809757 88.257992) (end 52.823096 88.257992) (width 0.2) (layer "F.Cu") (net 9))
 (segment (start 45.002654 65.874924) (end 45.002654 82.56355) (width 0.2) (layer "F.Cu") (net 7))
 (segment (start 45.002654 82.56355) (end 43.525654 84.04055) (width 0.2) (layer "F.Cu") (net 7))
 (segment (start 51.938336 58.939242) (end 45.002654 65.874924) (width 0.2) (layer "F.Cu") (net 7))
 (segment (start 118.283594 58.939242) (end 51.938336 58.939242) (width 0.2) (layer "F.Cu") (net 7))
 (segment (start 120.748944 61.404592) (end 118.283594 58.939242) (width 0.2) (layer "F.Cu") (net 7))
 (segment (start 125.76875 79.75125) (end 125.042492 79.024992) (width 0.2) (layer "B.Cu") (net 11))
 (segment (start 75.125454 61.9125) (end 74.494712 62.543242) (width 0.2) (layer "B.Cu") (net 11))
 (segment (start 125.042492 79.024992) (end 106.618214 79.024992) (width 0.2) (layer "B.Cu") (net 11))
 (segment (start 68.406712 62.543242) (end 67.77597 61.9125) (width 0.2) (layer "B.Cu") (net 11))
 (segment (start 74.494712 62.543242) (end 68.406712 62.543242) (width 0.2) (layer "B.Cu") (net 11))
 (segment (start 67.77597 61.9125) (end 42.8625 61.9125) (width 0.2) (layer "B.Cu") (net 11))
 (segment (start 41.08225 70.602146) (end 53.685654 83.20555) (width 0.2) (layer "B.Cu") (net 11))
 (segment (start 42.8625 61.9125) (end 41.08225 63.69275) (width 0.2) (layer "B.Cu") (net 11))
 (segment (start 89.505722 61.9125) (end 75.125454 61.9125) (width 0.2) (layer "B.Cu") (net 11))
 (segment (start 106.618214 79.024992) (end 89.505722 61.9125) (width 0.2) (layer "B.Cu") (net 11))
 (segment (start 41.08225 63.69275) (end 41.08225 70.602146) (width 0.2) (layer "B.Cu") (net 11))
 (segment (start 133.02 78.25125) (end 135.73125 80.9625) (width 0.2) (layer "B.Cu") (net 4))
 (segment (start 130.96875 78.25125) (end 133.02 78.25125) (width 0.2) (layer "B.Cu") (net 4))
 (segment (start 123.825 88.10625) (end 125.76875 88.10625) (width 0.2) (layer "B.Cu") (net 4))
 (segment (start 135.73125 80.9625) (end 135.73125 92.86875) (width 0.2) (layer "B.Cu") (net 4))
 (segment (start 135.73125 92.86875) (end 128.5875 92.86875) (width 0.2) (layer "B.Cu") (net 4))
 (segment (start 128.5875 92.86875) (end 123.825 88.10625) (width 0.2) (layer "B.Cu") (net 4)))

